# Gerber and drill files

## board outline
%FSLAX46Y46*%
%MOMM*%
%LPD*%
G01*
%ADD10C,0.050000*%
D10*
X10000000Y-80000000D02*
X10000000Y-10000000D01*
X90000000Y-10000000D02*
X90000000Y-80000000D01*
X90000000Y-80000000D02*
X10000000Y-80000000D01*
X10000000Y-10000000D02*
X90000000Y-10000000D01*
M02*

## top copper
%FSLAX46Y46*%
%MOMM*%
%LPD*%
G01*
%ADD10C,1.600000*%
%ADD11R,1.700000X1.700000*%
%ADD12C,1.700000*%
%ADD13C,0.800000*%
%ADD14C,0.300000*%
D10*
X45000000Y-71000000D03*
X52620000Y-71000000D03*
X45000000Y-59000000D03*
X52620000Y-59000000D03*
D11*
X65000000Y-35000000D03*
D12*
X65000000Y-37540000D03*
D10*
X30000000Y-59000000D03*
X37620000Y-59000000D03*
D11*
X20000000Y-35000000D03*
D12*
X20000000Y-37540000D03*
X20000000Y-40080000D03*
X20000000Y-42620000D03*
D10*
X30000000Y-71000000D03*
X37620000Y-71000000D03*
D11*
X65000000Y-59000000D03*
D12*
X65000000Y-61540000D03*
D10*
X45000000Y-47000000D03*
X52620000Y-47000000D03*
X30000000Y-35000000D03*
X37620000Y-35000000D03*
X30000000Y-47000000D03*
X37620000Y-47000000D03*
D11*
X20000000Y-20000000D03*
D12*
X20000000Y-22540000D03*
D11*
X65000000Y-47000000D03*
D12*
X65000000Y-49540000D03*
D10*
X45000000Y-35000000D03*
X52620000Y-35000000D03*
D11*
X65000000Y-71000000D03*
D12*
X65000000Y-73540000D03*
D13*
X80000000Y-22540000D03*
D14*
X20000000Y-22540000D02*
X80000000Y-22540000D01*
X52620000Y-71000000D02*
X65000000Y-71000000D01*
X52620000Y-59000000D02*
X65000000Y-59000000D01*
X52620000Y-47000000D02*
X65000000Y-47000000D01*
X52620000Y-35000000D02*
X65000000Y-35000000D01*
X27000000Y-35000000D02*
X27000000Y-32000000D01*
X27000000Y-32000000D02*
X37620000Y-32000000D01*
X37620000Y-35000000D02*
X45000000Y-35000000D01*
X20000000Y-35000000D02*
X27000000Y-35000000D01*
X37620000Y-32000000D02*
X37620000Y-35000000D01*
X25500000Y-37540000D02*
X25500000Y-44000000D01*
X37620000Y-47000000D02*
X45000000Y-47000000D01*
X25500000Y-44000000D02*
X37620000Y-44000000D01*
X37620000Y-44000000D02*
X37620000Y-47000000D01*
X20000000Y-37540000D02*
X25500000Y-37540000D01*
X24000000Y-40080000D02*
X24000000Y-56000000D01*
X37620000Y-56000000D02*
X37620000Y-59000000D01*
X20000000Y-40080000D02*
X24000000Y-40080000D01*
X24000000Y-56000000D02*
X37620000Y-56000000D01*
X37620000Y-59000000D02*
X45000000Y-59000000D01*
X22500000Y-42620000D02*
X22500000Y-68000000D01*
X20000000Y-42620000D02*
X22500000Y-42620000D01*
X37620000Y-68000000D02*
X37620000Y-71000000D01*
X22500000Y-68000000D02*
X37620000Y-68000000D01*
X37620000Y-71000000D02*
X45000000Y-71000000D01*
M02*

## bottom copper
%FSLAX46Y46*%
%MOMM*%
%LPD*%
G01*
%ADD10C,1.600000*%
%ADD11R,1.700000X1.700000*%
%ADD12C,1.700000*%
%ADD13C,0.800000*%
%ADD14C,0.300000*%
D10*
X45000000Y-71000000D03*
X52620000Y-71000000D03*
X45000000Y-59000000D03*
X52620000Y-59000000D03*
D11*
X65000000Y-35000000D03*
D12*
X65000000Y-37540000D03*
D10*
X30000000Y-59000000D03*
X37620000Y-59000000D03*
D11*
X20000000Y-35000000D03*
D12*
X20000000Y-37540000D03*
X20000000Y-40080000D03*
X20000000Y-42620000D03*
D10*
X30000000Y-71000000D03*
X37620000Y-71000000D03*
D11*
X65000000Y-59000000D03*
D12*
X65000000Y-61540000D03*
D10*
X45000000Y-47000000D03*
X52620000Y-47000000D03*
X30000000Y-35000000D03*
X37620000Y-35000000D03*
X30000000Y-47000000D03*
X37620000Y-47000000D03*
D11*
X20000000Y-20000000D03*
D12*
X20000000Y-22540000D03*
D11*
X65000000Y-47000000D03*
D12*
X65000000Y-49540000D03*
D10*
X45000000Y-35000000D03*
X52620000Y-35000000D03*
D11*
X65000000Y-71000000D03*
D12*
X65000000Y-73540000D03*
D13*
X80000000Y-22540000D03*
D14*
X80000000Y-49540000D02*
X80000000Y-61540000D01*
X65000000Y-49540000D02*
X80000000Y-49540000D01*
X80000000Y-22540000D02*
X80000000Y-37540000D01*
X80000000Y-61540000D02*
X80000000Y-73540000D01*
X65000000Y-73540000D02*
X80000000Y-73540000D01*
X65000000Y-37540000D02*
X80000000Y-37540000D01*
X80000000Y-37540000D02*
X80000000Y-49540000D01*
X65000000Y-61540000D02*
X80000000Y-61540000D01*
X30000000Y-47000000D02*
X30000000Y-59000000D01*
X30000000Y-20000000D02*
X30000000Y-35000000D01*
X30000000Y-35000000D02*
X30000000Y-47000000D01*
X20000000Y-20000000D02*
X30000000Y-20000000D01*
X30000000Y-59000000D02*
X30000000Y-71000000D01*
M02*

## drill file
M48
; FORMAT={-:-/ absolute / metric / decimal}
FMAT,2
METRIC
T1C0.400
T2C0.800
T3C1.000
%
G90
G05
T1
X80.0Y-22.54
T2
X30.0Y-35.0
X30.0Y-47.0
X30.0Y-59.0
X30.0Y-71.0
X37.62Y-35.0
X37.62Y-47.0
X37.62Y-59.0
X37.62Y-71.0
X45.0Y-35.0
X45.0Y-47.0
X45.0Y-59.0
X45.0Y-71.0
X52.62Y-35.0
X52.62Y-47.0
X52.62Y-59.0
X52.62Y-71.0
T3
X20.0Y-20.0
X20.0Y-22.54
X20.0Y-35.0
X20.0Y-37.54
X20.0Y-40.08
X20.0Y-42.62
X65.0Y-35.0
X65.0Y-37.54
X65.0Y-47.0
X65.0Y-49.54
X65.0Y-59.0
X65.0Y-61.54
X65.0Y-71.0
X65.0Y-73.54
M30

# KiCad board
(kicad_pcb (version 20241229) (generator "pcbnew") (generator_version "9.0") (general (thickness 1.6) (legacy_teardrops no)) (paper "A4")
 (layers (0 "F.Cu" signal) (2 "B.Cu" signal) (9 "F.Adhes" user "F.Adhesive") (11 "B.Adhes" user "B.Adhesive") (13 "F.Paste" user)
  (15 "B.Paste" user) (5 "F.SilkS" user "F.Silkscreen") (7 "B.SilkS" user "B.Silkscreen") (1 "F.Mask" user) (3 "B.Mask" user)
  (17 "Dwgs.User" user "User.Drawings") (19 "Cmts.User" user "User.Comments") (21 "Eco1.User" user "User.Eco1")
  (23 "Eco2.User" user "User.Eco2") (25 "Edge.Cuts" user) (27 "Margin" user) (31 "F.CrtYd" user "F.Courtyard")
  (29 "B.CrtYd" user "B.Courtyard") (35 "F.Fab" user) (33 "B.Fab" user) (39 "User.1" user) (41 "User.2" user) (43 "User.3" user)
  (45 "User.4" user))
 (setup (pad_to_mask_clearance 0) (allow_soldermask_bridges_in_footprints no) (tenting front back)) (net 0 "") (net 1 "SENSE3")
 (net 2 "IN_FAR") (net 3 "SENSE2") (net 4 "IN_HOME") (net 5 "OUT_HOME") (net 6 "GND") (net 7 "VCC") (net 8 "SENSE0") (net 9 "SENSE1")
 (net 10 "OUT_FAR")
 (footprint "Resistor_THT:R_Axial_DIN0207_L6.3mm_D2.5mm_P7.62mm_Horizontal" (layer "F.Cu") (at 45 71)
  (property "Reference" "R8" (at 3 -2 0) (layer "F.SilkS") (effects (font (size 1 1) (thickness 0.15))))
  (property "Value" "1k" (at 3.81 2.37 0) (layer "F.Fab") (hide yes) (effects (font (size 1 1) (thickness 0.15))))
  (pad "1" thru_hole circle (at 0 0) (size 1.6 1.6) (drill 0.8) (layers "*.Cu" "*.Mask") (remove_unused_layers no) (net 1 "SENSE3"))
  (pad "2" thru_hole circle (at 7.62 0) (size 1.6 1.6) (drill 0.8) (layers "*.Cu" "*.Mask") (remove_unused_layers no) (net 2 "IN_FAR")))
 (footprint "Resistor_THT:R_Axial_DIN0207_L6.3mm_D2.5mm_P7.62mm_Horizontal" (layer "F.Cu") (at 45 59)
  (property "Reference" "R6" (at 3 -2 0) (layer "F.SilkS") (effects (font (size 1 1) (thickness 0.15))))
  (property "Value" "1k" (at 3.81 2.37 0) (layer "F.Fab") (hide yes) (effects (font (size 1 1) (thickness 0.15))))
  (pad "1" thru_hole circle (at 0 0) (size 1.6 1.6) (drill 0.8) (layers "*.Cu" "*.Mask") (remove_unused_layers no) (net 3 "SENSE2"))
  (pad "2" thru_hole circle (at 7.62 0) (size 1.6 1.6) (drill 0.8) (layers "*.Cu" "*.Mask") (remove_unused_layers no) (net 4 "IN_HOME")))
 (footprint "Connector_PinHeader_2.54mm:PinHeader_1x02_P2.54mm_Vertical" (layer "F.Cu") (at 65 35)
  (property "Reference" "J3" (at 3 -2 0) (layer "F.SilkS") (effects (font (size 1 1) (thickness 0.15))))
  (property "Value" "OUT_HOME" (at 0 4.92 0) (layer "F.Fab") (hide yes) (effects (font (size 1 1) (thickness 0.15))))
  (pad "1" thru_hole rect (at 0 0) (size 1.7 1.7) (drill 1) (layers "*.Cu" "*.Mask") (remove_unused_layers no) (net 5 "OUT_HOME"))
  (pad "2" thru_hole circle (at 0 2.54) (size 1.7 1.7) (drill 1) (layers "*.Cu" "*.Mask") (remove_unused_layers no) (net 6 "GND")))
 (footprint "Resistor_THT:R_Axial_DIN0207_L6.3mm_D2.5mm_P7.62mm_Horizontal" (layer "F.Cu") (at 30 59)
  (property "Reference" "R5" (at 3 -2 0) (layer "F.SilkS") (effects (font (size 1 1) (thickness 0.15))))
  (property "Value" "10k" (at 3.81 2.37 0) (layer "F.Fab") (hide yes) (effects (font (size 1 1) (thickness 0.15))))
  (pad "1" thru_hole circle (at 0 0) (size 1.6 1.6) (drill 0.8) (layers "*.Cu" "*.Mask") (remove_unused_layers no) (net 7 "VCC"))
  (pad "2" thru_hole circle (at 7.62 0) (size 1.6 1.6) (drill 0.8) (layers "*.Cu" "*.Mask") (remove_unused_layers no) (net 3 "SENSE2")))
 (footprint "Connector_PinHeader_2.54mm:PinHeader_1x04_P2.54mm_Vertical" (layer "F.Cu") (at 20 35)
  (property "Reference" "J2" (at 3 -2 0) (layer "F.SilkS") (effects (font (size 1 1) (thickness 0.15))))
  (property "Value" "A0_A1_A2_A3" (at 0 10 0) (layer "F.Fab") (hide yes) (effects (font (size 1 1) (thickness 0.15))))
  (pad "1" thru_hole rect (at 0 0) (size 1.7 1.7) (drill 1) (layers "*.Cu" "*.Mask") (remove_unused_layers no) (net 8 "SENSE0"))
  (pad "2" thru_hole circle (at 0 2.54) (size 1.7 1.7) (drill 1) (layers "*.Cu" "*.Mask") (remove_unused_layers no) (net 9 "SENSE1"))
  (pad "3" thru_hole circle (at 0 5.08) (size 1.7 1.7) (drill 1) (layers "*.Cu" "*.Mask") (remove_unused_layers no) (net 3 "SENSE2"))
  (pad "4" thru_hole circle (at 0 7.62) (size 1.7 1.7) (drill 1) (layers "*.Cu" "*.Mask") (remove_unused_layers no) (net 1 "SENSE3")))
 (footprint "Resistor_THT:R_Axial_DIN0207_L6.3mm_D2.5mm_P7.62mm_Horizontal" (layer "F.Cu") (at 30 71)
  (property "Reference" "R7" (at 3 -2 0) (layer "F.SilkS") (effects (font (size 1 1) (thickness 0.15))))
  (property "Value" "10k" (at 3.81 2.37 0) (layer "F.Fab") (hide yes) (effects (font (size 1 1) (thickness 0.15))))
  (pad "1" thru_hole circle (at 0 0) (size 1.6 1.6) (drill 0.8) (layers "*.Cu" "*.Mask") (remove_unused_layers no) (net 7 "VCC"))
  (pad "2" thru_hole circle (at 7.62 0) (size 1.6 1.6) (drill 0.8) (layers "*.Cu" "*.Mask") (remove_unused_layers no) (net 1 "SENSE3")))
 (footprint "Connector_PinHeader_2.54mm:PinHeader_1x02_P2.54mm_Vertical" (layer "F.Cu") (at 65 59)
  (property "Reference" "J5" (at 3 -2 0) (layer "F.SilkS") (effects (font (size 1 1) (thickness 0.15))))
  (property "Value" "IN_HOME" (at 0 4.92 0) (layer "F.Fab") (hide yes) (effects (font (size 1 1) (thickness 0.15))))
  (pad "1" thru_hole rect (at 0 0) (size 1.7 1.7) (drill 1) (layers "*.Cu" "*.Mask") (remove_unused_layers no) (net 4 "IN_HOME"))
  (pad "2" thru_hole circle (at 0 2.54) (size 1.7 1.7) (drill 1) (layers "*.Cu" "*.Mask") (remove_unused_layers no) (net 6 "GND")))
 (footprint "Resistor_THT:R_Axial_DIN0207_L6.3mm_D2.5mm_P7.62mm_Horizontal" (layer "F.Cu") (at 45 47)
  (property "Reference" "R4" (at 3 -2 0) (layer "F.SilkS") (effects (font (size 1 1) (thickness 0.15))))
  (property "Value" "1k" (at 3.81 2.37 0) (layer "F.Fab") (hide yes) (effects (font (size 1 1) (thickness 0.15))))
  (pad "1" thru_hole circle (at 0 0) (size 1.6 1.6) (drill 0.8) (layers "*.Cu" "*.Mask") (remove_unused_layers no) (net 9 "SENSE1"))
  (pad "2" thru_hole circle (at 7.62 0) (size 1.6 1.6) (drill 0.8) (layers "*.Cu" "*.Mask") (remove_unused_layers no) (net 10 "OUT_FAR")))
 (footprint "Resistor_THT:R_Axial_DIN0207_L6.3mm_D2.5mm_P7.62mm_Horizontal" (layer "F.Cu") (at 30 35)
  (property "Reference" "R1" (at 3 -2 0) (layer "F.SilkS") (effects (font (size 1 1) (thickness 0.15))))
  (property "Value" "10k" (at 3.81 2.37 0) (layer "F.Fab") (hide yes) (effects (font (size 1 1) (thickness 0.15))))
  (pad "1" thru_hole circle (at 0 0) (size 1.6 1.6) (drill 0.8) (layers "*.Cu" "*.Mask") (remove_unused_layers no) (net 7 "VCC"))
  (pad "2" thru_hole circle (at 7.62 0) (size 1.6 1.6) (drill 0.8) (layers "*.Cu" "*.Mask") (remove_unused_layers no) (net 8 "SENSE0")))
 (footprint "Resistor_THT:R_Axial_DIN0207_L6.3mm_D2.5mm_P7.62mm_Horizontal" (layer "F.Cu") (at 30 47)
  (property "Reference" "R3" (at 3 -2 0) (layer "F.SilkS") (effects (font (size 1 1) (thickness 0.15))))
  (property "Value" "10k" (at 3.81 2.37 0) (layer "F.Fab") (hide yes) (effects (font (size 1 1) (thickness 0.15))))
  (pad "1" thru_hole circle (at 0 0) (size 1.6 1.6) (drill 0.8) (layers "*.Cu" "*.Mask") (remove_unused_layers no) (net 7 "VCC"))
  (pad "2" thru_hole circle (at 7.62 0) (size 1.6 1.6) (drill 0.8) (layers "*.Cu" "*.Mask") (remove_unused_layers no) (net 9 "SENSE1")))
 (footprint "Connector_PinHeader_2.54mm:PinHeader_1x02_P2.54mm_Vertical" (layer "F.Cu") (at 20 20)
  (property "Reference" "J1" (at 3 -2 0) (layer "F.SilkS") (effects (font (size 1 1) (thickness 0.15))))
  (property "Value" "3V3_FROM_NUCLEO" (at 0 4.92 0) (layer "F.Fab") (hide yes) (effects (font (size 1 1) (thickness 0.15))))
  (pad "1" thru_hole rect (at 0 0) (size 1.7 1.7) (drill 1) (layers "*.Cu" "*.Mask") (remove_unused_layers no) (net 7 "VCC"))
  (pad "2" thru_hole circle (at 0 2.54) (size 1.7 1.7) (drill 1) (layers "*.Cu" "*.Mask") (remove_unused_layers no) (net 6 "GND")))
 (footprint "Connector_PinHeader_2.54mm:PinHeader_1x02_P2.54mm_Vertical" (layer "F.Cu") (at 65 47)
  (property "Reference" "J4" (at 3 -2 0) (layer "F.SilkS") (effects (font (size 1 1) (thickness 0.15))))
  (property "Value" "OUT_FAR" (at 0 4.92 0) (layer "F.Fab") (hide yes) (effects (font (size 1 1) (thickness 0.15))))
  (pad "1" thru_hole rect (at 0 0) (size 1.7 1.7) (drill 1) (layers "*.Cu" "*.Mask") (remove_unused_layers no) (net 10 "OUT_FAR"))
  (pad "2" thru_hole circle (at 0 2.54) (size 1.7 1.7) (drill 1) (layers "*.Cu" "*.Mask") (remove_unused_layers no) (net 6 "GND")))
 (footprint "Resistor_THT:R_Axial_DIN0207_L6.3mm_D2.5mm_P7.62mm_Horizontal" (layer "F.Cu") (at 45 35)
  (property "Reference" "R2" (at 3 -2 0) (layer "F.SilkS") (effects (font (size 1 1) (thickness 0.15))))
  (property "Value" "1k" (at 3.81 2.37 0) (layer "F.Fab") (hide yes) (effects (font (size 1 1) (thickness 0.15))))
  (pad "1" thru_hole circle (at 0 0) (size 1.6 1.6) (drill 0.8) (layers "*.Cu" "*.Mask") (remove_unused_layers no) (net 8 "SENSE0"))
  (pad "2" thru_hole circle (at 7.62 0) (size 1.6 1.6) (drill 0.8) (layers "*.Cu" "*.Mask") (remove_unused_layers no) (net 5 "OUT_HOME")))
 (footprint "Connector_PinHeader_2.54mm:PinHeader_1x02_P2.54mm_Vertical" (layer "F.Cu") (at 65 71)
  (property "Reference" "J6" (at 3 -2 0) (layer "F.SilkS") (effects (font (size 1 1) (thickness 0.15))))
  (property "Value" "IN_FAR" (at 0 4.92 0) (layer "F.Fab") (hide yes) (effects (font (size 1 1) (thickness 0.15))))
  (pad "1" thru_hole rect (at 0 0) (size 1.7 1.7) (drill 1) (layers "*.Cu" "*.Mask") (remove_unused_layers no) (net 2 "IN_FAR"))
  (pad "2" thru_hole circle (at 0 2.54) (size 1.7 1.7) (drill 1) (layers "*.Cu" "*.Mask") (remove_unused_layers no) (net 6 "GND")))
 (gr_line (start 10 80) (end 10 10) (stroke (width 0.05) (type default)) (layer "Edge.Cuts"))
 (gr_line (start 90 10) (end 90 80) (stroke (width 0.05) (type default)) (layer "Edge.Cuts"))
 (gr_line (start 90 80) (end 10 80) (stroke (width 0.05) (type default)) (layer "Edge.Cuts"))
 (gr_line (start 10 10) (end 90 10) (stroke (width 0.05) (type default)) (layer "Edge.Cuts"))
 (segment (start 20 22.54) (end 80 22.54) (width 0.3) (layer "F.Cu") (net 6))
 (via (at 80 22.54) (size 0.8) (drill 0.4) (layers "F.Cu" "B.Cu") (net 6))
 (segment (start 80 49.54) (end 80 61.54) (width 0.3) (layer "B.Cu") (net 6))
 (segment (start 65 49.54) (end 80 49.54) (width 0.3) (layer "B.Cu") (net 6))
 (segment (start 80 22.54) (end 80 37.54) (width 0.3) (layer "B.Cu") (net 6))
 (segment (start 80 61.54) (end 80 73.54) (width 0.3) (layer "B.Cu") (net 6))
 (segment (start 65 73.54) (end 80 73.54) (width 0.3) (layer "B.Cu") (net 6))
 (segment (start 65 37.54) (end 80 37.54) (width 0.3) (layer "B.Cu") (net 6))
 (segment (start 80 37.54) (end 80 49.54) (width 0.3) (layer "B.Cu") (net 6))
 (segment (start 65 61.54) (end 80 61.54) (width 0.3) (layer "B.Cu") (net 6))
 (segment (start 52.62 71) (end 65 71) (width 0.3) (layer "F.Cu") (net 2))
 (segment (start 52.62 59) (end 65 59) (width 0.3) (layer "F.Cu") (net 4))
 (segment (start 52.62 47) (end 65 47) (width 0.3) (layer "F.Cu") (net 10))
 (segment (start 52.62 35) (end 65 35) (width 0.3) (layer "F.Cu") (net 5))
 (segment (start 27 35) (end 27 32) (width 0.3) (layer "F.Cu") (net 8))
 (segment (start 27 32) (end 37.62 32) (width 0.3) (layer "F.Cu") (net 8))
 (segment (start 37.62 35) (end 45 35) (width 0.3) (layer "F.Cu") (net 8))
 (segment (start 20 35) (end 27 35) (width 0.3) (layer "F.Cu") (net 8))
 (segment (start 37.62 32) (end 37.62 35) (width 0.3) (layer "F.Cu") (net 8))
 (segment (start 25.5 37.54) (end 25.5 44) (width 0.3) (layer "F.Cu") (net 9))
 (segment (start 37.62 47) (end 45 47) (width 0.3) (layer "F.Cu") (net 9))
 (segment (start 25.5 44) (end 37.62 44) (width 0.3) (layer "F.Cu") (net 9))
 (segment (start 37.62 44) (end 37.62 47) (width 0.3) (layer "F.Cu") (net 9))
 (segment (start 20 37.54) (end 25.5 37.54) (width 0.3) (layer "F.Cu") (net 9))
 (segment (start 24 40.08) (end 24 56) (width 0.3) (layer "F.Cu") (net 3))
 (segment (start 37.62 56) (end 37.62 59) (width 0.3) (layer "F.Cu") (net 3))
 (segment (start 20 40.08) (end 24 40.08) (width 0.3) (layer "F.Cu") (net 3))
 (segment (start 24 56) (end 37.62 56) (width 0.3) (layer "F.Cu") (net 3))
 (segment (start 37.62 59) (end 45 59) (width 0.3) (layer "F.Cu") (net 3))
 (segment (start 22.5 42.62) (end 22.5 68) (width 0.3) (layer "F.Cu") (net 1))
 (segment (start 20 42.62) (end 22.5 42.62) (width 0.3) (layer "F.Cu") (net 1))
 (segment (start 37.62 68) (end 37.62 71) (width 0.3) (layer "F.Cu") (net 1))
 (segment (start 22.5 68) (end 37.62 68) (width 0.3) (layer "F.Cu") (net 1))
 (segment (start 37.62 71) (end 45 71) (width 0.3) (layer "F.Cu") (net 1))
 (segment (start 30 47) (end 30 59) (width 0.3) (layer "B.Cu") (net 7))
 (segment (start 30 20) (end 30 35) (width 0.3) (layer "B.Cu") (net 7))
 (segment (start 30 35) (end 30 47) (width 0.3) (layer "B.Cu") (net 7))
 (segment (start 20 20) (end 30 20) (width 0.3) (layer "B.Cu") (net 7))
 (segment (start 30 59) (end 30 71) (width 0.3) (layer "B.Cu") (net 7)))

